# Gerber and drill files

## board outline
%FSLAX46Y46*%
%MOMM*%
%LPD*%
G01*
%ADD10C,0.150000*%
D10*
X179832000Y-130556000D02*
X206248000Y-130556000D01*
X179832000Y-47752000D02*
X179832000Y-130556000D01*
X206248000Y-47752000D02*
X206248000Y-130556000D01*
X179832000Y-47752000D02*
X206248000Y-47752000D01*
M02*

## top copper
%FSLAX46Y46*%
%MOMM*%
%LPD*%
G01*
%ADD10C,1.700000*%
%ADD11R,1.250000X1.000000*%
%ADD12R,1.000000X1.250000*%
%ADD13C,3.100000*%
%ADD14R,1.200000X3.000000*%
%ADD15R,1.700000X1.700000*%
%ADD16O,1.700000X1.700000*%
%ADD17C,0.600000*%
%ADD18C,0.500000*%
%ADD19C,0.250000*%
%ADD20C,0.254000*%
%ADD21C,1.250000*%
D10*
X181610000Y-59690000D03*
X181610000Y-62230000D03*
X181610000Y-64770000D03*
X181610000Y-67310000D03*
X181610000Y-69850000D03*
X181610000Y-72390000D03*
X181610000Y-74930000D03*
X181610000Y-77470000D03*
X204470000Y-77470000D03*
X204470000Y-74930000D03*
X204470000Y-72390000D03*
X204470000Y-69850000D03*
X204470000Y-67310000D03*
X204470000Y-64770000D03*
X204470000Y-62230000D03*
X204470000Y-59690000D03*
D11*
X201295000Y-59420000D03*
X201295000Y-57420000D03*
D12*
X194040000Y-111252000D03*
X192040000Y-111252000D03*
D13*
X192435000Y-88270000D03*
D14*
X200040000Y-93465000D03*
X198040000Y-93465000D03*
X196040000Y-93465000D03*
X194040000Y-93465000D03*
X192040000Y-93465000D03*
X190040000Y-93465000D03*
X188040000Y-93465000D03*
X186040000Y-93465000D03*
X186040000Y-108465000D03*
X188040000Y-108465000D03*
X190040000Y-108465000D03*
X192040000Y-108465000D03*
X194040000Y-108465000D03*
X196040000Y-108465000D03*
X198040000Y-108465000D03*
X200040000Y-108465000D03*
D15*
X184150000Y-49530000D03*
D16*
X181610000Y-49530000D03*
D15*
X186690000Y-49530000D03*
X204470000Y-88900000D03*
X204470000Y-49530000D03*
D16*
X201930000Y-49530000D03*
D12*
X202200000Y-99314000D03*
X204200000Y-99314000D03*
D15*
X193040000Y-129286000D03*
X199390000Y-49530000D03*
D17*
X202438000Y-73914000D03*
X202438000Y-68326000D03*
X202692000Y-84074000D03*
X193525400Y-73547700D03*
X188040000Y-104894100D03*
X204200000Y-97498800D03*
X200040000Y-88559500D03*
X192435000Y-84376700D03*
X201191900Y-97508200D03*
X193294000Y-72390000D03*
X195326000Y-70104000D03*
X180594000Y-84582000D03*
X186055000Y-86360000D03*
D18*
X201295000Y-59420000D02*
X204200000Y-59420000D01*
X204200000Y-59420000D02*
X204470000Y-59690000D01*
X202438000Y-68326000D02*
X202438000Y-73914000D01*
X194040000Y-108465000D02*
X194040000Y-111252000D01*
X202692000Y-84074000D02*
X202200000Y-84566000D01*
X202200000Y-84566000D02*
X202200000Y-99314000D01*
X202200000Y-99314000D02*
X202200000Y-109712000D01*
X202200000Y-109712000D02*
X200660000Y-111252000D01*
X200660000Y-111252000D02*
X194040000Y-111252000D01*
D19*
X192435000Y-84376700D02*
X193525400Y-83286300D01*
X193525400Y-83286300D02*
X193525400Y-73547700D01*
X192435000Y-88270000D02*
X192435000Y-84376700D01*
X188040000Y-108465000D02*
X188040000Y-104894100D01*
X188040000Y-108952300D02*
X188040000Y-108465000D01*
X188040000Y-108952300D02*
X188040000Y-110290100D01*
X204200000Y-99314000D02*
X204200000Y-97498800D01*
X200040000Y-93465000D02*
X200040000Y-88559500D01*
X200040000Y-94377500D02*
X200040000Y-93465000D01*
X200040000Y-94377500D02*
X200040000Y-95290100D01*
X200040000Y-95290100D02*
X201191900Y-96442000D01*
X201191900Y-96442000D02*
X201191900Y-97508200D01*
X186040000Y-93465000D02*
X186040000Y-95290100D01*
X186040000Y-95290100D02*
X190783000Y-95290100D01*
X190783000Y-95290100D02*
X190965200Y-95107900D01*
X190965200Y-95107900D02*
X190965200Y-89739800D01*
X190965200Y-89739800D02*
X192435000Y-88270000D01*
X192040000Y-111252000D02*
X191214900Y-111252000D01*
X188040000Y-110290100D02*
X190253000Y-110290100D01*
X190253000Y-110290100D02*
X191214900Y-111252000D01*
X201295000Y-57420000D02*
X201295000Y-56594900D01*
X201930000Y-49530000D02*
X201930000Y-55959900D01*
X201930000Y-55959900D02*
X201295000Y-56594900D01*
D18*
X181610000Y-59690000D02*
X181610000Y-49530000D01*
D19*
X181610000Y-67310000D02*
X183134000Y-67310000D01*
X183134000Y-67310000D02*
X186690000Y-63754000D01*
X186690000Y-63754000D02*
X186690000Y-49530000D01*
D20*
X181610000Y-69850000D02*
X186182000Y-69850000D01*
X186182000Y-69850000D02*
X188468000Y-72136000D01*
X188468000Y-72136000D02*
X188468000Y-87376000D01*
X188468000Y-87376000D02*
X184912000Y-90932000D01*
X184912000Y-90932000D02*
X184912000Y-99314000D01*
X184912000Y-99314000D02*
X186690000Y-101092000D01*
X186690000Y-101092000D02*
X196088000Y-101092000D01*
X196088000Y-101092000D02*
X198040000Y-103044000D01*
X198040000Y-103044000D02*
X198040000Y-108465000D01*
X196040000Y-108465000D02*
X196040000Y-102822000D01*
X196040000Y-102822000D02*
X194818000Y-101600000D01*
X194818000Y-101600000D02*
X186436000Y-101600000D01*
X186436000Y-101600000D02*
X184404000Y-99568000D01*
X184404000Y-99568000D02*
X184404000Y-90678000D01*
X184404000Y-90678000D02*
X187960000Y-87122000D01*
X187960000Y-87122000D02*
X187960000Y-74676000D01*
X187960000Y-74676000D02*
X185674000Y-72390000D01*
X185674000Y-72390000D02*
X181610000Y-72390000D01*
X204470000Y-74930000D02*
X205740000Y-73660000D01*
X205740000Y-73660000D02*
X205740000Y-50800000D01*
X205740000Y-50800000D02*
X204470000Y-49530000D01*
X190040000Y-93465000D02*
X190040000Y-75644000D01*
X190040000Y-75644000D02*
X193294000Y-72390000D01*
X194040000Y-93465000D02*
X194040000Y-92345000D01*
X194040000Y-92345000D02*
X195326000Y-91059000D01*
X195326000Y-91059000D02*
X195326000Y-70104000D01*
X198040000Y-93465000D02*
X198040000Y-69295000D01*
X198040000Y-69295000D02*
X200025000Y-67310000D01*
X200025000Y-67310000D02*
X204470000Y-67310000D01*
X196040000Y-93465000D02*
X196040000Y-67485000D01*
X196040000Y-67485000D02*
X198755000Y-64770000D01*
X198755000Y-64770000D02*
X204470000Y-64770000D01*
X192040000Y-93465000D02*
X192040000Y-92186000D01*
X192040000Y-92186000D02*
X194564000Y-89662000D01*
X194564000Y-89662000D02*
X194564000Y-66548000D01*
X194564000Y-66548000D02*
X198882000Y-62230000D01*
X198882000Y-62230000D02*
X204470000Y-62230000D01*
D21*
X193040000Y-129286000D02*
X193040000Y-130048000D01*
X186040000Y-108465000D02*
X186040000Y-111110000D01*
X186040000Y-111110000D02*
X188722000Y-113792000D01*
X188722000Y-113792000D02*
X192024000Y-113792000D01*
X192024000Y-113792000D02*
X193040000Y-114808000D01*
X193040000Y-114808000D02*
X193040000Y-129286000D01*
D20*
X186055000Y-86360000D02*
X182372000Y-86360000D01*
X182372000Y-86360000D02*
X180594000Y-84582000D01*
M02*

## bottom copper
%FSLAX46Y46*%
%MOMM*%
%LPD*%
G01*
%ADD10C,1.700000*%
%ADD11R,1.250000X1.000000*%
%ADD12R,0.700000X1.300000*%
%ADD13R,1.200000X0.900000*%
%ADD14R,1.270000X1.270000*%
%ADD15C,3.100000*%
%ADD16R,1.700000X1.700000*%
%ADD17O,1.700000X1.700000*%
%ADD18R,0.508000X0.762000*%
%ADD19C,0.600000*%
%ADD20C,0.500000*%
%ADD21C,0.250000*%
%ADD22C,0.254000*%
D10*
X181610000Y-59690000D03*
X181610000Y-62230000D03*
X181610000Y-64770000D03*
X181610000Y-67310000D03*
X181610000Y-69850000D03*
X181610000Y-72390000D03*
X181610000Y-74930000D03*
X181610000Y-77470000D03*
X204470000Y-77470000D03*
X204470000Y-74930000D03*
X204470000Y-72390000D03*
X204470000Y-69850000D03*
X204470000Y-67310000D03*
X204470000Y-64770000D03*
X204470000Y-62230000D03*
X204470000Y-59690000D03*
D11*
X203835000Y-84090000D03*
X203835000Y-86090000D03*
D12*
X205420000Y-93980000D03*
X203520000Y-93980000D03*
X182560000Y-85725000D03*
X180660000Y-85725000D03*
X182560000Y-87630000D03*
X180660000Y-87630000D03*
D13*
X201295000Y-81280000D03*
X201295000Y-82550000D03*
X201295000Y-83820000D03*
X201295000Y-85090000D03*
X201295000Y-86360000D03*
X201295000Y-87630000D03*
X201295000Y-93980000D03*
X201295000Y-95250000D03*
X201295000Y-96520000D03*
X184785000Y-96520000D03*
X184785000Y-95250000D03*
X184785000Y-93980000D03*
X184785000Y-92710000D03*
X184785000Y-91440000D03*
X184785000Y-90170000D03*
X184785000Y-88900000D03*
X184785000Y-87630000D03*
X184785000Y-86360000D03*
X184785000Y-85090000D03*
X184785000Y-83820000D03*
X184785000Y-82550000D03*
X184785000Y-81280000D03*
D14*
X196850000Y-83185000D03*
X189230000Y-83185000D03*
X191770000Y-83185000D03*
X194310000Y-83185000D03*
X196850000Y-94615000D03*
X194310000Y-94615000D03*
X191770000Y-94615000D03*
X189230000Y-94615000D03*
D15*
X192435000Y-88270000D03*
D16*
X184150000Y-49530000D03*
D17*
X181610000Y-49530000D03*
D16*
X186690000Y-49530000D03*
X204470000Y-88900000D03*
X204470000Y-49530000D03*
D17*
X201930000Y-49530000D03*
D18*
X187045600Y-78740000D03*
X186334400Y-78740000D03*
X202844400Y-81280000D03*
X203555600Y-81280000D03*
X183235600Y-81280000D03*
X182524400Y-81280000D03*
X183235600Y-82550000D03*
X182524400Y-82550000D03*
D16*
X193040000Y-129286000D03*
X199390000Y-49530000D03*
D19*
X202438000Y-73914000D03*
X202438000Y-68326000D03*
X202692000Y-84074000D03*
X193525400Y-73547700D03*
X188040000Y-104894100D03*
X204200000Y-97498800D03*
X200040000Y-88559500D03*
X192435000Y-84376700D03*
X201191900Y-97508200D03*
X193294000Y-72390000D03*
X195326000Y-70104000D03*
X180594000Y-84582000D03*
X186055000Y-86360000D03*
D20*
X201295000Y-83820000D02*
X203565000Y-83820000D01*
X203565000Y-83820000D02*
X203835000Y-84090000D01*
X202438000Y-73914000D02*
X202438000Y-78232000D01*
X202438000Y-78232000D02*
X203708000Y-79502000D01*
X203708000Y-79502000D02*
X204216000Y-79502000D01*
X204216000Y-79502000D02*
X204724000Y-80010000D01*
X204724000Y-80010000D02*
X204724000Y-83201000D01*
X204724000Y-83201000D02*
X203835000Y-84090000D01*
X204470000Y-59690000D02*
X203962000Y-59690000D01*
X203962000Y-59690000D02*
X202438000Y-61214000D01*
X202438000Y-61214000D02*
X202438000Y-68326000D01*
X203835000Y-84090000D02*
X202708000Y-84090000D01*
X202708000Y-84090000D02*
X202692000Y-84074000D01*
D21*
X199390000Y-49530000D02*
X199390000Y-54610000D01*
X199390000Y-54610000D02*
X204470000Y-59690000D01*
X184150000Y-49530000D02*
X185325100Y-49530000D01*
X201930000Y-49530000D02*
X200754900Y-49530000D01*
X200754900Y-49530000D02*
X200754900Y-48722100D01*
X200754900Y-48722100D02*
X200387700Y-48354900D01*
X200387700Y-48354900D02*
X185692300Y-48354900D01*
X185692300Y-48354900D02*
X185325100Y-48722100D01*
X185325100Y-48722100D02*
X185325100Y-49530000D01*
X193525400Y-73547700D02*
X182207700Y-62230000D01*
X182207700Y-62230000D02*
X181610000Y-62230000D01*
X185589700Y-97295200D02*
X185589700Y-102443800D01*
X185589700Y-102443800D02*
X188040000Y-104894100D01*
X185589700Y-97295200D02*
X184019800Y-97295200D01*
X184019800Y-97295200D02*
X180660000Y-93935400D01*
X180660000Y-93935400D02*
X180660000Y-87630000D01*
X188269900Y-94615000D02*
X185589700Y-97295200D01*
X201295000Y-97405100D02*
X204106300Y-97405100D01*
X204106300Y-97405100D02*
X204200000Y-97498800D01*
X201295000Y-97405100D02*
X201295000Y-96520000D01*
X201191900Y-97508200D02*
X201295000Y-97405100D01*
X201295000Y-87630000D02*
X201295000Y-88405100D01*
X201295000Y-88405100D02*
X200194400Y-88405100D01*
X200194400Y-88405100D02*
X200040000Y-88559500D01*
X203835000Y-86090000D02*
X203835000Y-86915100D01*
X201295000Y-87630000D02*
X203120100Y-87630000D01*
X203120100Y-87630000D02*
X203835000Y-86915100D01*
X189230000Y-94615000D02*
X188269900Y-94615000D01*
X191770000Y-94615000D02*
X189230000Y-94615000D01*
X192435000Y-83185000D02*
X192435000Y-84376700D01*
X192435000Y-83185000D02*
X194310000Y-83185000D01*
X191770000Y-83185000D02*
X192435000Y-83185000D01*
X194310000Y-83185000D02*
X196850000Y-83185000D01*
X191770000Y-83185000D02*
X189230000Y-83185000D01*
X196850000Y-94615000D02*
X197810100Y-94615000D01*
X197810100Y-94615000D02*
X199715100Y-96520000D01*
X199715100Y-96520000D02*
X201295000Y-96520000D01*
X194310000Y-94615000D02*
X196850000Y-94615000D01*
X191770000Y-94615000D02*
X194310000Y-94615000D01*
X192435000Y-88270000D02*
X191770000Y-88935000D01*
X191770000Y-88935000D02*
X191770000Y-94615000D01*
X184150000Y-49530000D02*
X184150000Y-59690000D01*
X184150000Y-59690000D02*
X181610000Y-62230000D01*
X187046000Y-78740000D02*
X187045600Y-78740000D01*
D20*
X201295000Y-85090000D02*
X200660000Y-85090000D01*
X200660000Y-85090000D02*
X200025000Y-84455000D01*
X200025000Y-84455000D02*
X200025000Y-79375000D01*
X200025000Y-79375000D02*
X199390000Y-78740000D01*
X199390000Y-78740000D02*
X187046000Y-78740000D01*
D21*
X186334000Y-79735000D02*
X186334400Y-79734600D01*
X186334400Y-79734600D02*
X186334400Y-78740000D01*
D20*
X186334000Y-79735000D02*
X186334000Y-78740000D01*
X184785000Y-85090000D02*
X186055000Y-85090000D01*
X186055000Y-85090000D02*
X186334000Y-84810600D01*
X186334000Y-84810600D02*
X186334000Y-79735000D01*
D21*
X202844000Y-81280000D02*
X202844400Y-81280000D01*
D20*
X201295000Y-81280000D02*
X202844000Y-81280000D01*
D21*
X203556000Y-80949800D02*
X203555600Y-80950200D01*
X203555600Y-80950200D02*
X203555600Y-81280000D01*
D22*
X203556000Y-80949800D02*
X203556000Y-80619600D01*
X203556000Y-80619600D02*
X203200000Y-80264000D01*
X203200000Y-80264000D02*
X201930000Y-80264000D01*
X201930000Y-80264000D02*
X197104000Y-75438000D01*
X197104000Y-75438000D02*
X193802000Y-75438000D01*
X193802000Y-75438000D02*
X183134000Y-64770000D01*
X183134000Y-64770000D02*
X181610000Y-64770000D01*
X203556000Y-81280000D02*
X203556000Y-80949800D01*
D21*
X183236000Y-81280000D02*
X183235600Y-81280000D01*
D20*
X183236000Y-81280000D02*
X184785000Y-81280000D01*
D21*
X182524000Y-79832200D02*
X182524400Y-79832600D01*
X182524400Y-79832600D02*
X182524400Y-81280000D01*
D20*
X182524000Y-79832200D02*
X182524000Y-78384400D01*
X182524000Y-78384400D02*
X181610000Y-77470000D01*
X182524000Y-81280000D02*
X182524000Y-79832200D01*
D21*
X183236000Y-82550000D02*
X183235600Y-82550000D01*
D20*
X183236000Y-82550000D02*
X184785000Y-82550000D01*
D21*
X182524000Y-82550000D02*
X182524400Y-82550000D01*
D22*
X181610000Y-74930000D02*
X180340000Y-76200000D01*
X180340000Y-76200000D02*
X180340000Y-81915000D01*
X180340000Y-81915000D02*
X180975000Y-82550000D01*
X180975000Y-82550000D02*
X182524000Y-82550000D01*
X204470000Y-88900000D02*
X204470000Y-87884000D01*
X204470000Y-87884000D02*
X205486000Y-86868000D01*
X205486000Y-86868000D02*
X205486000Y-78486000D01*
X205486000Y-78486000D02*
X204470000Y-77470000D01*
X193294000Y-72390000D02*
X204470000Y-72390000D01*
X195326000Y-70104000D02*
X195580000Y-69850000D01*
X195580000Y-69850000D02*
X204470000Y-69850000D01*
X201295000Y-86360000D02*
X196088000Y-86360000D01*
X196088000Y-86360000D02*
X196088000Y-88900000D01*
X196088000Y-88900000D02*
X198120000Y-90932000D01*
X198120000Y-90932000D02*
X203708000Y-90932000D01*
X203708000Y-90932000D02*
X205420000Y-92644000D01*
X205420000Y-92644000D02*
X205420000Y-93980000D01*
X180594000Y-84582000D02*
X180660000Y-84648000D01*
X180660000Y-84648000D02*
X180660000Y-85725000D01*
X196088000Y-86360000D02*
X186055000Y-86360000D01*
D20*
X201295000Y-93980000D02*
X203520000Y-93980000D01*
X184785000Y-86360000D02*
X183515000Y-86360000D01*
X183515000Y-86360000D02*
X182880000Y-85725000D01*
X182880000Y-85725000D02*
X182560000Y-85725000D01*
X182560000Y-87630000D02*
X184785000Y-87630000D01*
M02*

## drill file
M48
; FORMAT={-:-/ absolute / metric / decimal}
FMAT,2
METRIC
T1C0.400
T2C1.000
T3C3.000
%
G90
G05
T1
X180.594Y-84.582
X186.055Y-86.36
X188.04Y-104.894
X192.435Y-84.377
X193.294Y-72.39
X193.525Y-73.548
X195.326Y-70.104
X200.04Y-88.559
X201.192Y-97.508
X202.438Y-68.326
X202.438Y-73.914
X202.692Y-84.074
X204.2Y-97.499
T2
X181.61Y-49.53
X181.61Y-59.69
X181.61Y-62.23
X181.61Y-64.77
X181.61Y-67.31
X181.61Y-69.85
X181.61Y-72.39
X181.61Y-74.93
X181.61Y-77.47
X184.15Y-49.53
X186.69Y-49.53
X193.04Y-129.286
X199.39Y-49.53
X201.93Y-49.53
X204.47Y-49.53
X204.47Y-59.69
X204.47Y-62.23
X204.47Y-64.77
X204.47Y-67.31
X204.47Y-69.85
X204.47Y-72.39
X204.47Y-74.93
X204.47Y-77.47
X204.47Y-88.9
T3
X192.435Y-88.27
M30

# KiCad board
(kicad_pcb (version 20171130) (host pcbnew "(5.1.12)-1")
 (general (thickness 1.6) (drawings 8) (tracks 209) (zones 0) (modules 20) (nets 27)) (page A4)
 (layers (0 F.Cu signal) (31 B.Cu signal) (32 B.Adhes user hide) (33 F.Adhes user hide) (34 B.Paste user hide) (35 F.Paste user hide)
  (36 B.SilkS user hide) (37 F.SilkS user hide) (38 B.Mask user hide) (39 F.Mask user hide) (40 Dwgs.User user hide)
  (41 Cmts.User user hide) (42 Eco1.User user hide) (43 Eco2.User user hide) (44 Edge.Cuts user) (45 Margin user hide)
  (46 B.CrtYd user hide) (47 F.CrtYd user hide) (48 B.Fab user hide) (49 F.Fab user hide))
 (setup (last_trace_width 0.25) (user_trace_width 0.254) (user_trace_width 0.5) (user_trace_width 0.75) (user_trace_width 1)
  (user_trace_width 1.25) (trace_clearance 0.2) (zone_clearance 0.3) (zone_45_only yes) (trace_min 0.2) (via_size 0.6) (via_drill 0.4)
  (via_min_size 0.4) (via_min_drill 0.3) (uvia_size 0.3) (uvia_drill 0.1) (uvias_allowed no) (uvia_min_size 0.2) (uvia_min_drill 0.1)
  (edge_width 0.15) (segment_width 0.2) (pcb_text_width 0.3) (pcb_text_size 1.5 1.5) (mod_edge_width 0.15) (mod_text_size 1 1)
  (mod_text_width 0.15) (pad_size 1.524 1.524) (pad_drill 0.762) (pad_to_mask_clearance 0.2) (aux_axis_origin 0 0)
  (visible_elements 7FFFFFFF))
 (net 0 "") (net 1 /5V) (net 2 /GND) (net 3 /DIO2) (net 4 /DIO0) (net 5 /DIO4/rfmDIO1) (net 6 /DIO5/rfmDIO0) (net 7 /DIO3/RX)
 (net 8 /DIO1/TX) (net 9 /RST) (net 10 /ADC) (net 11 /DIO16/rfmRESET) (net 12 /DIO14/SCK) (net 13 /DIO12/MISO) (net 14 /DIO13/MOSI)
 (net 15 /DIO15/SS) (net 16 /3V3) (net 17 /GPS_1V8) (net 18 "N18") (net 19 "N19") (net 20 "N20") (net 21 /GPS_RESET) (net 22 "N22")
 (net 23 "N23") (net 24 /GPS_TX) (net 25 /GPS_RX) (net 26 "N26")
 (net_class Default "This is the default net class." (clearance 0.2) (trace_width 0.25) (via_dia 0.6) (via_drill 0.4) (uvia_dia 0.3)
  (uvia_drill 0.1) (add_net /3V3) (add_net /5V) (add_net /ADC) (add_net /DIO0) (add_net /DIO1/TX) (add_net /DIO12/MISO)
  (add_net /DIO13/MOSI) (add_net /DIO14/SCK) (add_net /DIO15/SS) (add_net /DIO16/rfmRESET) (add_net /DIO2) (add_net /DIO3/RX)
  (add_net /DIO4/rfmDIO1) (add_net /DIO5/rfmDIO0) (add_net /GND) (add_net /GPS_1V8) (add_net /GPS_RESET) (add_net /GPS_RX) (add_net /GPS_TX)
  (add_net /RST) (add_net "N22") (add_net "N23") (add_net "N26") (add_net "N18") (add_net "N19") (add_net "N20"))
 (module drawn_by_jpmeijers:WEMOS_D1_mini (layer F.Cu) (at 193.04 68.58)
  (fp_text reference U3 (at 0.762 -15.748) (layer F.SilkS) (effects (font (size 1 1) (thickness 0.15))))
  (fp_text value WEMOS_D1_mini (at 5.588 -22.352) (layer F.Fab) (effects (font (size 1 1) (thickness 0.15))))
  (pad 1 thru_hole circle (at -11.43 -8.89) (size 1.7 1.7) (drill 1) (layers *.Cu *.Mask) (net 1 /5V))
  (pad 2 thru_hole circle (at -11.43 -6.35) (size 1.7 1.7) (drill 1) (layers *.Cu *.Mask) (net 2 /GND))
  (pad 3 thru_hole circle (at -11.43 -3.81) (size 1.7 1.7) (drill 1) (layers *.Cu *.Mask) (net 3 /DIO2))
  (pad 4 thru_hole circle (at -11.43 -1.27) (size 1.7 1.7) (drill 1) (layers *.Cu *.Mask) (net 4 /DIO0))
  (pad 5 thru_hole circle (at -11.43 1.27) (size 1.7 1.7) (drill 1) (layers *.Cu *.Mask) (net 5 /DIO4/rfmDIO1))
  (pad 6 thru_hole circle (at -11.43 3.81) (size 1.7 1.7) (drill 1) (layers *.Cu *.Mask) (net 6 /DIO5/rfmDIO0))
  (pad 7 thru_hole circle (at -11.43 6.35) (size 1.7 1.7) (drill 1) (layers *.Cu *.Mask) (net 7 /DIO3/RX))
  (pad 8 thru_hole circle (at -11.43 8.89) (size 1.7 1.7) (drill 1) (layers *.Cu *.Mask) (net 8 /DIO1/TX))
  (pad 9 thru_hole circle (at 11.43 8.89) (size 1.7 1.7) (drill 1) (layers *.Cu *.Mask) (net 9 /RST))
  (pad 10 thru_hole circle (at 11.43 6.35) (size 1.7 1.7) (drill 1) (layers *.Cu *.Mask) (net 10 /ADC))
  (pad 11 thru_hole circle (at 11.43 3.81) (size 1.7 1.7) (drill 1) (layers *.Cu *.Mask) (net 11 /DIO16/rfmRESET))
  (pad 12 thru_hole circle (at 11.43 1.27) (size 1.7 1.7) (drill 1) (layers *.Cu *.Mask) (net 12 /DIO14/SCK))
  (pad 13 thru_hole circle (at 11.43 -1.27) (size 1.7 1.7) (drill 1) (layers *.Cu *.Mask) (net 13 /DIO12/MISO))
  (pad 14 thru_hole circle (at 11.43 -3.81) (size 1.7 1.7) (drill 1) (layers *.Cu *.Mask) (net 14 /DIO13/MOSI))
  (pad 15 thru_hole circle (at 11.43 -6.35) (size 1.7 1.7) (drill 1) (layers *.Cu *.Mask) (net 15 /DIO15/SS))
  (pad 16 thru_hole circle (at 11.43 -8.89) (size 1.7 1.7) (drill 1) (layers *.Cu *.Mask) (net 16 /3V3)))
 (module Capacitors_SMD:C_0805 (layer F.Cu) (at 201.295 58.42 90)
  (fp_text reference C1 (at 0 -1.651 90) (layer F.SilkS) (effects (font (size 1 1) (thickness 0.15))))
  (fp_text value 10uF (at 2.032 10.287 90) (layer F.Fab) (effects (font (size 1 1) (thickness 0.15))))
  (pad 1 smd rect (at -1 0 90) (size 1 1.25) (layers F.Cu F.Paste F.Mask) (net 16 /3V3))
  (pad 2 smd rect (at 1 0 90) (size 1 1.25) (layers F.Cu F.Paste F.Mask) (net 2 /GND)))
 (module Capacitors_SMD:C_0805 (layer B.Cu) (at 203.835 85.09 270)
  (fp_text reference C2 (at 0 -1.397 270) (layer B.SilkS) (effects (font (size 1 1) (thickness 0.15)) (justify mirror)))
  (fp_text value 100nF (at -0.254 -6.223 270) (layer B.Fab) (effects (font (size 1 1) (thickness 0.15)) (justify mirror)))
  (pad 1 smd rect (at -1 0 270) (size 1 1.25) (layers B.Cu B.Paste B.Mask) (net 16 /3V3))
  (pad 2 smd rect (at 1 0 270) (size 1 1.25) (layers B.Cu B.Paste B.Mask) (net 2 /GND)))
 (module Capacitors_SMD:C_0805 (layer F.Cu) (at 193.04 111.252 180)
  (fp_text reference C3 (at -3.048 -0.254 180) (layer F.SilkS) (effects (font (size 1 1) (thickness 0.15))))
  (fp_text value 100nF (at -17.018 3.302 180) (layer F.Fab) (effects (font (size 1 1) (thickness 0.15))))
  (pad 1 smd rect (at -1 0 180) (size 1 1.25) (layers F.Cu F.Paste F.Mask) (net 16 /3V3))
  (pad 2 smd rect (at 1 0 180) (size 1 1.25) (layers F.Cu F.Paste F.Mask) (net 2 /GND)))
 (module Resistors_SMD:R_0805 (layer B.Cu) (at 204.47 93.98 180)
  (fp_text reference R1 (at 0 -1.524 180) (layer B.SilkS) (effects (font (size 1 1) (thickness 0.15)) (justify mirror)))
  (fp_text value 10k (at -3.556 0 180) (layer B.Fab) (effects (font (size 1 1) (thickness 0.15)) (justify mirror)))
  (pad 1 smd rect (at -0.95 0 180) (size 0.7 1.3) (layers B.Cu B.Paste B.Mask) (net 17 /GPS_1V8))
  (pad 2 smd rect (at 0.95 0 180) (size 0.7 1.3) (layers B.Cu B.Paste B.Mask) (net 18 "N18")))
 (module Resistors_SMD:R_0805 (layer B.Cu) (at 181.61 85.725 180)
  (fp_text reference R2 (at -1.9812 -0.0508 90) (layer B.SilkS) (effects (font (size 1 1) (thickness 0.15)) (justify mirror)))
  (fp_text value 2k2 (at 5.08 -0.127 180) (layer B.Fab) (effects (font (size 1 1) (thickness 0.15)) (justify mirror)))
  (pad 1 smd rect (at -0.95 0 180) (size 0.7 1.3) (layers B.Cu B.Paste B.Mask) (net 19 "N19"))
  (pad 2 smd rect (at 0.95 0 180) (size 0.7 1.3) (layers B.Cu B.Paste B.Mask) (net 17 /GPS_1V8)))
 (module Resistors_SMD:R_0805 (layer B.Cu) (at 181.61 87.63 180)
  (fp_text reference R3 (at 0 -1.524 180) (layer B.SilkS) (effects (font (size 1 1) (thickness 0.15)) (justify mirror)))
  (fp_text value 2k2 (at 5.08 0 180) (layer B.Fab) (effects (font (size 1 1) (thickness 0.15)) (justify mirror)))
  (pad 1 smd rect (at -0.95 0 180) (size 0.7 1.3) (layers B.Cu B.Paste B.Mask) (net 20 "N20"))
  (pad 2 smd rect (at 0.95 0 180) (size 0.7 1.3) (layers B.Cu B.Paste B.Mask) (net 2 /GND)))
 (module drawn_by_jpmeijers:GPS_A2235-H (layer B.Cu) (at 201.295 97.79 180)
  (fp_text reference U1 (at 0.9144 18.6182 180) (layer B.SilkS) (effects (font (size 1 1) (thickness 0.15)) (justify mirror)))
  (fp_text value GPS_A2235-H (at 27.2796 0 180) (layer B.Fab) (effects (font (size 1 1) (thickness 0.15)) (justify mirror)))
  (pad 1 smd rect (at 0 16.51 180) (size 1.2 0.9) (layers B.Cu B.Paste B.Mask) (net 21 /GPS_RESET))
  (pad 2 smd rect (at 0 15.24 180) (size 1.2 0.9) (layers B.Cu B.Paste B.Mask))
  (pad 3 smd rect (at 0 13.97 180) (size 1.2 0.9) (layers B.Cu B.Paste B.Mask) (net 16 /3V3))
  (pad 4 smd rect (at 0 12.7 180) (size 1.2 0.9) (layers B.Cu B.Paste B.Mask) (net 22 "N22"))
  (pad 5 smd rect (at 0 11.43 180) (size 1.2 0.9) (layers B.Cu B.Paste B.Mask) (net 17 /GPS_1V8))
  (pad 6 smd rect (at 0 10.16 180) (size 1.2 0.9) (layers B.Cu B.Paste B.Mask) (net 2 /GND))
  (pad 7 smd rect (at 0 3.81 180) (size 1.2 0.9) (layers B.Cu B.Paste B.Mask) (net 18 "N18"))
  (pad 8 smd rect (at 0 2.54 180) (size 1.2 0.9) (layers B.Cu B.Paste B.Mask))
  (pad 9 smd rect (at 0 1.27 180) (size 1.2 0.9) (layers B.Cu B.Paste B.Mask) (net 2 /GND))
  (pad 10 smd rect (at 16.51 1.27 180) (size 1.2 0.9) (layers B.Cu B.Paste B.Mask))
  (pad 11 smd rect (at 16.51 2.54 180) (size 1.2 0.9) (layers B.Cu B.Paste B.Mask))
  (pad 12 smd rect (at 16.51 3.81 180) (size 1.2 0.9) (layers B.Cu B.Paste B.Mask))
  (pad 13 smd rect (at 16.51 5.08 180) (size 1.2 0.9) (layers B.Cu B.Paste B.Mask))
  (pad 14 smd rect (at 16.51 6.35 180) (size 1.2 0.9) (layers B.Cu B.Paste B.Mask))
  (pad 15 smd rect (at 16.51 7.62 180) (size 1.2 0.9) (layers B.Cu B.Paste B.Mask))
  (pad 16 smd rect (at 16.51 8.89 180) (size 1.2 0.9) (layers B.Cu B.Paste B.Mask))
  (pad 17 smd rect (at 16.51 10.16 180) (size 1.2 0.9) (layers B.Cu B.Paste B.Mask) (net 20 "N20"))
  (pad 18 smd rect (at 16.51 11.43 180) (size 1.2 0.9) (layers B.Cu B.Paste B.Mask) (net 19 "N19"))
  (pad 19 smd rect (at 16.51 12.7 180) (size 1.2 0.9) (layers B.Cu B.Paste B.Mask) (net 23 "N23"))
  (pad 20 smd rect (at 16.51 13.97 180) (size 1.2 0.9) (layers B.Cu B.Paste B.Mask))
  (pad 21 smd rect (at 16.51 15.24 180) (size 1.2 0.9) (layers B.Cu B.Paste B.Mask) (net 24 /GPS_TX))
  (pad 22 smd rect (at 16.51 16.51 180) (size 1.2 0.9) (layers B.Cu B.Paste B.Mask) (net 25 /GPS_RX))
  (pad 23 smd rect (at 4.445 14.605 180) (size 1.27 1.27) (layers B.Cu B.Paste B.Mask) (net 2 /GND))
  (pad 26 smd rect (at 12.065 14.605 180) (size 1.27 1.27) (layers B.Cu B.Paste B.Mask) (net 2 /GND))
  (pad 25 smd rect (at 9.525 14.605 180) (size 1.27 1.27) (layers B.Cu B.Paste B.Mask) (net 2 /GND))
  (pad 24 smd rect (at 6.985 14.605 180) (size 1.27 1.27) (layers B.Cu B.Paste B.Mask) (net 2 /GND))
  (pad 27 smd rect (at 4.445 3.175 180) (size 1.27 1.27) (layers B.Cu B.Paste B.Mask) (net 2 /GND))
  (pad 28 smd rect (at 6.985 3.175 180) (size 1.27 1.27) (layers B.Cu B.Paste B.Mask) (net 2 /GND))
  (pad 29 smd rect (at 9.525 3.175 180) (size 1.27 1.27) (layers B.Cu B.Paste B.Mask) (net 2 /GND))
  (pad 30 smd rect (at 12.065 3.175 180) (size 1.27 1.27) (layers B.Cu B.Paste B.Mask) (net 2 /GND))
  (pad 31 thru_hole circle (at 8.86 9.52 180) (size 3.1 3.1) (drill 3) (layers *.Cu *.Mask B.SilkS) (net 2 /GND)))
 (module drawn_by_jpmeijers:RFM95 (layer F.Cu) (at 193.04 100.965 270)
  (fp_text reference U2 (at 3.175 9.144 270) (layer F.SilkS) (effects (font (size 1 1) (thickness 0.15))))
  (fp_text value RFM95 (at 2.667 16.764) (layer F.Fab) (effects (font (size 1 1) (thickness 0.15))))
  (pad 1 smd rect (at -7.5 -7 270) (size 3 1.2) (layers F.Cu F.Paste F.Mask) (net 2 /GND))
  (pad 2 smd rect (at -7.5 -5 270) (size 3 1.2) (layers F.Cu F.Paste F.Mask) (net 13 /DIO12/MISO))
  (pad 3 smd rect (at -7.5 -3 270) (size 3 1.2) (layers F.Cu F.Paste F.Mask) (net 14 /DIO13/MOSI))
  (pad 4 smd rect (at -7.5 -1 270) (size 3 1.2) (layers F.Cu F.Paste F.Mask) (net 12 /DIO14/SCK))
  (pad 5 smd rect (at -7.5 1 270) (size 3 1.2) (layers F.Cu F.Paste F.Mask) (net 15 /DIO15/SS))
  (pad 6 smd rect (at -7.5 3 270) (size 3 1.2) (layers F.Cu F.Paste F.Mask) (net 11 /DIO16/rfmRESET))
  (pad 7 smd rect (at -7.5 5 270) (size 3 1.2) (layers F.Cu F.Paste F.Mask))
  (pad 8 smd rect (at -7.5 7 270) (size 3 1.2) (layers F.Cu F.Paste F.Mask) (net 2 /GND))
  (pad 9 smd rect (at 7.5 7 270) (size 3 1.2) (layers F.Cu F.Paste F.Mask) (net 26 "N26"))
  (pad 10 smd rect (at 7.5 5 270) (size 3 1.2) (layers F.Cu F.Paste F.Mask) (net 2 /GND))
  (pad 11 smd rect (at 7.5 3 270) (size 3 1.2) (layers F.Cu F.Paste F.Mask))
  (pad 12 smd rect (at 7.5 1 270) (size 3 1.2) (layers F.Cu F.Paste F.Mask))
  (pad 13 smd rect (at 7.5 -1 270) (size 3 1.2) (layers F.Cu F.Paste F.Mask) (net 16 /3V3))
  (pad 14 smd rect (at 7.5 -3 270) (size 3 1.2) (layers F.Cu F.Paste F.Mask) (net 6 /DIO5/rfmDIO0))
  (pad 15 smd rect (at 7.5 -5 270) (size 3 1.2) (layers F.Cu F.Paste F.Mask) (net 5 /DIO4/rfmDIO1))
  (pad 16 smd rect (at 7.5 -7 270) (size 3 1.2) (layers F.Cu F.Paste F.Mask)))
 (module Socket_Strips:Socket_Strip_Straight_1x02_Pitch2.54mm (layer F.Cu) (at 184.15 49.53 270)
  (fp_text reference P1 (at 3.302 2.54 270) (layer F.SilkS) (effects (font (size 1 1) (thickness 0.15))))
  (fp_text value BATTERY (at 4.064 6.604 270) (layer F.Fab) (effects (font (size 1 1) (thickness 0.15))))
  (pad 1 thru_hole rect (at 0 0 270) (size 1.7 1.7) (drill 1) (layers *.Cu *.Mask) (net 2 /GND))
  (pad 2 thru_hole oval (at 0 2.54 270) (size 1.7 1.7) (drill 1) (layers *.Cu *.Mask) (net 1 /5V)))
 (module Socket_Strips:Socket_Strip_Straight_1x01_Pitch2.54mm (layer F.Cu) (at 186.69 49.53)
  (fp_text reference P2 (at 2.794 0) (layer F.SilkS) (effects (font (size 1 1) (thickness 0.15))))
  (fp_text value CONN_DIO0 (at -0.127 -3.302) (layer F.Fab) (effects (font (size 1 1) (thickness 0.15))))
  (pad 1 thru_hole rect (at 0 0) (size 1.7 1.7) (drill 1) (layers *.Cu *.Mask) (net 4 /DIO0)))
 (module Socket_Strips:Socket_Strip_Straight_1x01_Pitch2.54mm (layer F.Cu) (at 204.47 88.9)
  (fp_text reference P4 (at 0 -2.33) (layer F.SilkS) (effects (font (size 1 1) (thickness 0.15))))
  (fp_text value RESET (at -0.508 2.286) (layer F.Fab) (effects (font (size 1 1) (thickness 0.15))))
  (pad 1 thru_hole rect (at 0 0) (size 1.7 1.7) (drill 1) (layers *.Cu *.Mask) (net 9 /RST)))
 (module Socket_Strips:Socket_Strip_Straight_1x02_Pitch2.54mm (layer F.Cu) (at 204.47 49.53 270)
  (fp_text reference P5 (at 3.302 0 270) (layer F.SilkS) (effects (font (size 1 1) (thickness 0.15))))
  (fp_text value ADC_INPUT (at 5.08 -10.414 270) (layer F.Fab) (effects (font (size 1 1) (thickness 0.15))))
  (pad 1 thru_hole rect (at 0 0 270) (size 1.7 1.7) (drill 1) (layers *.Cu *.Mask) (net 10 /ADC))
  (pad 2 thru_hole oval (at 0 2.54 270) (size 1.7 1.7) (drill 1) (layers *.Cu *.Mask) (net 2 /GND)))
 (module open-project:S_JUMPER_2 (layer B.Cu) (at 186.69 78.74 180)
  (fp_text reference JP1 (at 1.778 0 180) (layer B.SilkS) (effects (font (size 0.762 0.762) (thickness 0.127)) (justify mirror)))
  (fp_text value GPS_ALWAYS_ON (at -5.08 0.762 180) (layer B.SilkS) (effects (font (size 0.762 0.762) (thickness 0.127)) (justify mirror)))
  (pad 1 smd rect (at -0.3556 0 180) (size 0.508 0.762) (layers B.Cu B.Paste B.Mask) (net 22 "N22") (clearance 0.2032))
  (pad 2 smd rect (at 0.3556 0 180) (size 0.508 0.762) (layers B.Cu B.Paste B.Mask) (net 23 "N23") (clearance 0.2032)))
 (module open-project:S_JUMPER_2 (layer B.Cu) (at 203.2 81.28)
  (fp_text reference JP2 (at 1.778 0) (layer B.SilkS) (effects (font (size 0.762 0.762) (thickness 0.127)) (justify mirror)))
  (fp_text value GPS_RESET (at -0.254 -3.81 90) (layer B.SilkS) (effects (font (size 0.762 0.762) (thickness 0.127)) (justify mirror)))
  (pad 1 smd rect (at -0.3556 0) (size 0.508 0.762) (layers B.Cu B.Paste B.Mask) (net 21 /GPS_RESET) (clearance 0.2032))
  (pad 2 smd rect (at 0.3556 0) (size 0.508 0.762) (layers B.Cu B.Paste B.Mask) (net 3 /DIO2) (clearance 0.2032)))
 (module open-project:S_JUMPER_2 (layer B.Cu) (at 182.88 81.28 180)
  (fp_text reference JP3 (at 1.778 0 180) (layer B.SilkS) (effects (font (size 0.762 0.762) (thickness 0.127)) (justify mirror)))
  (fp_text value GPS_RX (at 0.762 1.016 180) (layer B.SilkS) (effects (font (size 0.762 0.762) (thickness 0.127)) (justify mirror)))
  (pad 1 smd rect (at -0.3556 0 180) (size 0.508 0.762) (layers B.Cu B.Paste B.Mask) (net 25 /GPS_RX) (clearance 0.2032))
  (pad 2 smd rect (at 0.3556 0 180) (size 0.508 0.762) (layers B.Cu B.Paste B.Mask) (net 8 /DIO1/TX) (clearance 0.2032)))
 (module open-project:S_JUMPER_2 (layer B.Cu) (at 182.88 82.55 180)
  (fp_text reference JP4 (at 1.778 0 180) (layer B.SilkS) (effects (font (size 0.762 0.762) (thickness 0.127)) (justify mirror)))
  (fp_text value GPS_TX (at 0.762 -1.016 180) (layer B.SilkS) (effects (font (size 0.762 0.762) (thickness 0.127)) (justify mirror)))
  (pad 1 smd rect (at -0.3556 0 180) (size 0.508 0.762) (layers B.Cu B.Paste B.Mask) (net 24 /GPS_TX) (clearance 0.2032))
  (pad 2 smd rect (at 0.3556 0 180) (size 0.508 0.762) (layers B.Cu B.Paste B.Mask) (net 7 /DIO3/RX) (clearance 0.2032)))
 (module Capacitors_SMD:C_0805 (layer F.Cu) (at 203.2 99.314)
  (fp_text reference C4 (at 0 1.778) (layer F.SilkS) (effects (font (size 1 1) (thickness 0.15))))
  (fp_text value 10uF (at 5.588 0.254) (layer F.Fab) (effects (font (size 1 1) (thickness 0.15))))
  (pad 1 smd rect (at -1 0) (size 1 1.25) (layers F.Cu F.Paste F.Mask) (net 16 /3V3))
  (pad 2 smd rect (at 1 0) (size 1 1.25) (layers F.Cu F.Paste F.Mask) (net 2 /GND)))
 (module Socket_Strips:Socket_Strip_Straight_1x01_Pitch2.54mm (layer F.Cu) (at 193.04 129.286)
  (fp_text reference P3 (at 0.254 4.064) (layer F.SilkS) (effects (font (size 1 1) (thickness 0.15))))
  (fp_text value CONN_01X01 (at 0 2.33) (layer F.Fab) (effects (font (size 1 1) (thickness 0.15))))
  (pad 1 thru_hole rect (at 0 0) (size 1.7 1.7) (drill 1) (layers *.Cu *.Mask) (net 26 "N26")))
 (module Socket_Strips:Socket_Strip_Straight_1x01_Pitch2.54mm (layer F.Cu) (at 199.39 49.53)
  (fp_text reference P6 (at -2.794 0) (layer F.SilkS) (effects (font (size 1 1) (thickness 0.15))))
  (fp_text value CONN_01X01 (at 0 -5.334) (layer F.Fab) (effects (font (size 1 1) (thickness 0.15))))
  (pad 1 thru_hole rect (at 0 0) (size 1.7 1.7) (drill 1) (layers *.Cu *.Mask) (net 16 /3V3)))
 (gr_line (start 179.832 130.556) (end 206.248 130.556) (angle 90) (layer Edge.Cuts) (width 0.15))
 (gr_line (start 179.832 47.752) (end 179.832 130.556) (angle 90) (layer Edge.Cuts) (width 0.15))
 (gr_line (start 206.248 47.752) (end 206.248 130.556) (angle 90) (layer Edge.Cuts) (width 0.15))
 (gr_line (start 179.832 47.752) (end 206.248 47.752) (angle 90) (layer Edge.Cuts) (width 0.15))
 (segment (start 201.295 83.82) (end 203.565 83.82) (width 0.5) (layer B.Cu) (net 16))
 (segment (start 203.565 83.82) (end 203.835 84.09) (width 0.5) (layer B.Cu) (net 16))
 (segment (start 201.295 59.42) (end 204.2 59.42) (width 0.5) (layer F.Cu) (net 16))
 (segment (start 204.2 59.42) (end 204.47 59.69) (width 0.5) (layer F.Cu) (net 16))
 (segment (start 202.438 73.914) (end 202.438 78.232) (width 0.5) (layer B.Cu) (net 16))
 (segment (start 202.438 78.232) (end 203.708 79.502) (width 0.5) (layer B.Cu) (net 16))
 (segment (start 203.708 79.502) (end 204.216 79.502) (width 0.5) (layer B.Cu) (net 16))
 (segment (start 204.216 79.502) (end 204.724 80.01) (width 0.5) (layer B.Cu) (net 16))
 (segment (start 204.724 80.01) (end 204.724 83.201) (width 0.5) (layer B.Cu) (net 16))
 (segment (start 204.724 83.201) (end 203.835 84.09) (width 0.5) (layer B.Cu) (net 16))
 (segment (start 202.438 68.326) (end 202.438 73.914) (width 0.5) (layer F.Cu) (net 16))
 (segment (start 204.47 59.69) (end 203.962 59.69) (width 0.5) (layer B.Cu) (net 16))
 (segment (start 203.962 59.69) (end 202.438 61.214) (width 0.5) (layer B.Cu) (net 16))
 (segment (start 202.438 61.214) (end 202.438 68.326) (width 0.5) (layer B.Cu) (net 16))
 (segment (start 194.04 108.465) (end 194.04 111.252) (width 0.5) (layer F.Cu) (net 16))
 (segment (start 203.835 84.09) (end 202.708 84.09) (width 0.5) (layer B.Cu) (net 16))
 (segment (start 202.708 84.09) (end 202.692 84.074) (width 0.5) (layer B.Cu) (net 16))
 (segment (start 202.692 84.074) (end 202.2 84.566) (width 0.5) (layer F.Cu) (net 16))
 (segment (start 202.2 84.566) (end 202.2 99.314) (width 0.5) (layer F.Cu) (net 16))
 (segment (start 202.2 99.314) (end 202.2 109.712) (width 0.5) (layer F.Cu) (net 16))
 (segment (start 202.2 109.712) (end 200.66 111.252) (width 0.5) (layer F.Cu) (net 16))
 (segment (start 200.66 111.252) (end 194.04 111.252) (width 0.5) (layer F.Cu) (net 16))
 (segment (start 199.39 49.53) (end 199.39 54.61) (width 0.25) (layer B.Cu) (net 16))
 (segment (start 199.39 54.61) (end 204.47 59.69) (width 0.25) (layer B.Cu) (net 16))
 (via (at 202.438 73.914) (size 0.6) (layers F.Cu B.Cu) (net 16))
 (via (at 202.438 68.326) (size 0.6) (layers F.Cu B.Cu) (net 16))
 (via (at 202.692 84.074) (size 0.6) (layers F.Cu B.Cu) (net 16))
 (segment (start 184.15 49.53) (end 185.3251 49.53) (width 0.25) (layer B.Cu) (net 2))
 (segment (start 201.93 49.53) (end 200.7549 49.53) (width 0.25) (layer B.Cu) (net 2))
 (segment (start 200.7549 49.53) (end 200.7549 48.7221) (width 0.25) (layer B.Cu) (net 2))
 (segment (start 200.7549 48.7221) (end 200.3877 48.3549) (width 0.25) (layer B.Cu) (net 2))
 (segment (start 200.3877 48.3549) (end 185.6923 48.3549) (width 0.25) (layer B.Cu) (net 2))
 (segment (start 185.6923 48.3549) (end 185.3251 48.7221) (width 0.25) (layer B.Cu) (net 2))
 (segment (start 185.3251 48.7221) (end 185.3251 49.53) (width 0.25) (layer B.Cu) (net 2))
 (segment (start 192.435 84.3767) (end 193.5254 83.2863) (width 0.25) (layer F.Cu) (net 2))
 (segment (start 193.5254 83.2863) (end 193.5254 73.5477) (width 0.25) (layer F.Cu) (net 2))
 (segment (start 192.435 88.27) (end 192.435 84.3767) (width 0.25) (layer F.Cu) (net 2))
 (segment (start 193.5254 73.5477) (end 182.2077 62.23) (width 0.25) (layer B.Cu) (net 2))
 (segment (start 182.2077 62.23) (end 181.61 62.23) (width 0.25) (layer B.Cu) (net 2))
 (segment (start 188.04 108.465) (end 188.04 104.8941) (width 0.25) (layer F.Cu) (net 2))
 (segment (start 185.5897 97.2952) (end 185.5897 102.4438) (width 0.25) (layer B.Cu) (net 2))
 (segment (start 185.5897 102.4438) (end 188.04 104.8941) (width 0.25) (layer B.Cu) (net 2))
 (segment (start 185.5897 97.2952) (end 184.0198 97.2952) (width 0.25) (layer B.Cu) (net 2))
 (segment (start 184.0198 97.2952) (end 180.66 93.9354) (width 0.25) (layer B.Cu) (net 2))
 (segment (start 180.66 93.9354) (end 180.66 87.63) (width 0.25) (layer B.Cu) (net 2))
 (segment (start 188.2699 94.615) (end 185.5897 97.2952) (width 0.25) (layer B.Cu) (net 2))
 (segment (start 188.04 108.9523) (end 188.04 108.465) (width 0.25) (layer F.Cu) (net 2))
 (segment (start 188.04 108.9523) (end 188.04 110.2901) (width 0.25) (layer F.Cu) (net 2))
 (segment (start 204.2 99.314) (end 204.2 97.4988) (width 0.25) (layer F.Cu) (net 2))
 (segment (start 201.295 97.4051) (end 204.1063 97.4051) (width 0.25) (layer B.Cu) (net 2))
 (segment (start 204.1063 97.4051) (end 204.2 97.4988) (width 0.25) (layer B.Cu) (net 2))
 (segment (start 201.295 97.4051) (end 201.295 96.52) (width 0.25) (layer B.Cu) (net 2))
 (segment (start 201.1919 97.5082) (end 201.295 97.4051) (width 0.25) (layer B.Cu) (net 2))
 (segment (start 201.295 87.63) (end 201.295 88.4051) (width 0.25) (layer B.Cu) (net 2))
 (segment (start 200.04 93.465) (end 200.04 88.5595) (width 0.25) (layer F.Cu) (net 2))
 (segment (start 201.295 88.4051) (end 200.1944 88.4051) (width 0.25) (layer B.Cu) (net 2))
 (segment (start 200.1944 88.4051) (end 200.04 88.5595) (width 0.25) (layer B.Cu) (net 2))
 (segment (start 200.04 94.3775) (end 200.04 93.465) (width 0.25) (layer F.Cu) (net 2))
 (segment (start 200.04 94.3775) (end 200.04 95.2901) (width 0.25) (layer F.Cu) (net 2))
 (segment (start 203.835 86.09) (end 203.835 86.9151) (width 0.25) (layer B.Cu) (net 2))
 (segment (start 201.295 87.63) (end 203.1201 87.63) (width 0.25) (layer B.Cu) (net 2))
 (segment (start 203.1201 87.63) (end 203.835 86.9151) (width 0.25) (layer B.Cu) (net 2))
 (segment (start 189.23 94.615) (end 188.2699 94.615) (width 0.25) (layer B.Cu) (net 2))
 (segment (start 191.77 94.615) (end 189.23 94.615) (width 0.25) (layer B.Cu) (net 2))
 (segment (start 192.435 83.185) (end 192.435 84.3767) (width 0.25) (layer B.Cu) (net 2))
 (segment (start 192.435 83.185) (end 194.31 83.185) (width 0.25) (layer B.Cu) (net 2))
 (segment (start 191.77 83.185) (end 192.435 83.185) (width 0.25) (layer B.Cu) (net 2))
 (segment (start 194.31 83.185) (end 196.85 83.185) (width 0.25) (layer B.Cu) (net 2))
 (segment (start 191.77 83.185) (end 189.23 83.185) (width 0.25) (layer B.Cu) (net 2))
 (segment (start 196.85 94.615) (end 197.8101 94.615) (width 0.25) (layer B.Cu) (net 2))
 (segment (start 197.8101 94.615) (end 199.7151 96.52) (width 0.25) (layer B.Cu) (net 2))
 (segment (start 199.7151 96.52) (end 201.295 96.52) (width 0.25) (layer B.Cu) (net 2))
 (segment (start 194.31 94.615) (end 196.85 94.615) (width 0.25) (layer B.Cu) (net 2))
 (segment (start 191.77 94.615) (end 194.31 94.615) (width 0.25) (layer B.Cu) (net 2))
 (segment (start 192.435 88.27) (end 191.77 88.935) (width 0.25) (layer B.Cu) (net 2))
 (segment (start 191.77 88.935) (end 191.77 94.615) (width 0.25) (layer B.Cu) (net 2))
 (segment (start 200.04 95.2901) (end 201.1919 96.442) (width 0.25) (layer F.Cu) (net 2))
 (segment (start 201.1919 96.442) (end 201.1919 97.5082) (width 0.25) (layer F.Cu) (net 2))
 (segment (start 186.04 93.465) (end 186.04 95.2901) (width 0.25) (layer F.Cu) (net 2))
 (segment (start 186.04 95.2901) (end 190.783 95.2901) (width 0.25) (layer F.Cu) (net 2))
 (segment (start 190.783 95.2901) (end 190.9652 95.1079) (width 0.25) (layer F.Cu) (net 2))
 (segment (start 190.9652 95.1079) (end 190.9652 89.7398) (width 0.25) (layer F.Cu) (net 2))
 (segment (start 190.9652 89.7398) (end 192.435 88.27) (width 0.25) (layer F.Cu) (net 2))
 (segment (start 192.04 111.252) (end 191.2149 111.252) (width 0.25) (layer F.Cu) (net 2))
 (segment (start 188.04 110.2901) (end 190.253 110.2901) (width 0.25) (layer F.Cu) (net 2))
 (segment (start 190.253 110.2901) (end 191.2149 111.252) (width 0.25) (layer F.Cu) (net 2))
 (segment (start 184.15 49.53) (end 184.15 59.69) (width 0.25) (layer B.Cu) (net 2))
 (segment (start 184.15 59.69) (end 181.61 62.23) (width 0.25) (layer B.Cu) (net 2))
 (segment (start 201.295 57.42) (end 201.295 56.5949) (width 0.25) (layer F.Cu) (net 2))
 (segment (start 201.93 49.53) (end 201.93 55.9599) (width 0.25) (layer F.Cu) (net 2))
 (segment (start 201.93 55.9599) (end 201.295 56.5949) (width 0.25) (layer F.Cu) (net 2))
 (via (at 193.5254 73.5477) (size 0.6) (layers F.Cu B.Cu) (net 2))
 (via (at 188.04 104.8941) (size 0.6) (layers F.Cu B.Cu) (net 2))
 (via (at 204.2 97.4988) (size 0.6) (layers F.Cu B.Cu) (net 2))
 (via (at 200.04 88.5595) (size 0.6) (layers F.Cu B.Cu) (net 2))
 (via (at 192.435 84.3767) (size 0.6) (layers F.Cu B.Cu) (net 2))
 (via (at 201.1919 97.5082) (size 0.6) (layers F.Cu B.Cu) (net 2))
 (segment (start 187.046 78.74) (end 187.0456 78.74) (width 0.25) (layer B.Cu) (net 22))
 (segment (start 201.295 85.09) (end 200.66 85.09) (width 0.5) (layer B.Cu) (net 22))
 (segment (start 200.66 85.09) (end 200.025 84.455) (width 0.5) (layer B.Cu) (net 22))
 (segment (start 200.025 84.455) (end 200.025 79.375) (width 0.5) (layer B.Cu) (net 22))
 (segment (start 200.025 79.375) (end 199.39 78.74) (width 0.5) (layer B.Cu) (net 22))
 (segment (start 199.39 78.74) (end 187.046 78.74) (width 0.5) (layer B.Cu) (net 22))
 (segment (start 186.334 79.735) (end 186.3344 79.7346) (width 0.25) (layer B.Cu) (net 23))
 (segment (start 186.3344 79.7346) (end 186.3344 78.74) (width 0.25) (layer B.Cu) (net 23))
 (segment (start 186.334 79.735) (end 186.334 78.74) (width 0.5) (layer B.Cu) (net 23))
 (segment (start 184.785 85.09) (end 186.055 85.09) (width 0.5) (layer B.Cu) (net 23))
 (segment (start 186.055 85.09) (end 186.334 84.8106) (width 0.5) (layer B.Cu) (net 23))
 (segment (start 186.334 84.8106) (end 186.334 79.735) (width 0.5) (layer B.Cu) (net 23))
 (segment (start 202.844 81.28) (end 202.8444 81.28) (width 0.25) (layer B.Cu) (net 21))
 (segment (start 201.295 81.28) (end 202.844 81.28) (width 0.5) (layer B.Cu) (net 21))
 (segment (start 203.556 80.9498) (end 203.5556 80.9502) (width 0.25) (layer B.Cu) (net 3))
 (segment (start 203.5556 80.9502) (end 203.5556 81.28) (width 0.25) (layer B.Cu) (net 3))
 (segment (start 203.556 80.9498) (end 203.556 80.6196) (width 0.254) (layer B.Cu) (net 3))
 (segment (start 203.556 80.6196) (end 203.2 80.264) (width 0.254) (layer B.Cu) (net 3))
 (segment (start 203.2 80.264) (end 201.93 80.264) (width 0.254) (layer B.Cu) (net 3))
 (segment (start 201.93 80.264) (end 197.104 75.438) (width 0.254) (layer B.Cu) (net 3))
 (segment (start 197.104 75.438) (end 193.802 75.438) (width 0.254) (layer B.Cu) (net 3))
 (segment (start 193.802 75.438) (end 183.134 64.77) (width 0.254) (layer B.Cu) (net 3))
 (segment (start 183.134 64.77) (end 181.61 64.77) (width 0.254) (layer B.Cu) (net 3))
 (segment (start 203.556 81.28) (end 203.556 80.9498) (width 0.254) (layer B.Cu) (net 3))
 (segment (start 183.236 81.28) (end 183.2356 81.28) (width 0.25) (layer B.Cu) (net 25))
 (segment (start 183.236 81.28) (end 184.785 81.28) (width 0.5) (layer B.Cu) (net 25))
 (segment (start 182.524 79.8322) (end 182.5244 79.8326) (width 0.25) (layer B.Cu) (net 8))
 (segment (start 182.5244 79.8326) (end 182.5244 81.28) (width 0.25) (layer B.Cu) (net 8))
 (segment (start 182.524 79.8322) (end 182.524 78.3844) (width 0.5) (layer B.Cu) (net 8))
 (segment (start 182.524 78.3844) (end 181.61 77.47) (width 0.5) (layer B.Cu) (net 8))
 (segment (start 182.524 81.28) (end 182.524 79.8322) (width 0.5) (layer B.Cu) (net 8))
 (segment (start 183.236 82.55) (end 183.2356 82.55) (width 0.25) (layer B.Cu) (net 24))
 (segment (start 183.236 82.55) (end 184.785 82.55) (width 0.5) (layer B.Cu) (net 24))
 (segment (start 182.524 82.55) (end 182.5244 82.55) (width 0.25) (layer B.Cu) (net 7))
 (segment (start 181.61 74.93) (end 180.34 76.2) (width 0.254) (layer B.Cu) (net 7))
 (segment (start 180.34 76.2) (end 180.34 81.915) (width 0.254) (layer B.Cu) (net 7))
 (segment (start 180.34 81.915) (end 180.975 82.55) (width 0.254) (layer B.Cu) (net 7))
 (segment (start 180.975 82.55) (end 182.524 82.55) (width 0.254) (layer B.Cu) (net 7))
 (segment (start 181.61 59.69) (end 181.61 49.53) (width 0.5) (layer F.Cu) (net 1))
 (segment (start 181.61 67.31) (end 183.134 67.31) (width 0.25) (layer F.Cu) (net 4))
 (segment (start 183.134 67.31) (end 186.69 63.754) (width 0.25) (layer F.Cu) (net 4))
 (segment (start 186.69 63.754) (end 186.69 49.53) (width 0.25) (layer F.Cu) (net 4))
 (segment (start 181.61 69.85) (end 186.182 69.85) (width 0.254) (layer F.Cu) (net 5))
 (segment (start 186.182 69.85) (end 188.468 72.136) (width 0.254) (layer F.Cu) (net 5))
 (segment (start 188.468 72.136) (end 188.468 87.376) (width 0.254) (layer F.Cu) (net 5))
 (segment (start 188.468 87.376) (end 184.912 90.932) (width 0.254) (layer F.Cu) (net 5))
 (segment (start 184.912 90.932) (end 184.912 99.314) (width 0.254) (layer F.Cu) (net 5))
 (segment (start 184.912 99.314) (end 186.69 101.092) (width 0.254) (layer F.Cu) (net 5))
 (segment (start 186.69 101.092) (end 196.088 101.092) (width 0.254) (layer F.Cu) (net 5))
 (segment (start 196.088 101.092) (end 198.04 103.044) (width 0.254) (layer F.Cu) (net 5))
 (segment (start 198.04 103.044) (end 198.04 108.465) (width 0.254) (layer F.Cu) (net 5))
 (segment (start 196.04 108.465) (end 196.04 102.822) (width 0.254) (layer F.Cu) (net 6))
 (segment (start 196.04 102.822) (end 194.818 101.6) (width 0.254) (layer F.Cu) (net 6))
 (segment (start 194.818 101.6) (end 186.436 101.6) (width 0.254) (layer F.Cu) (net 6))
 (segment (start 186.436 101.6) (end 184.404 99.568) (width 0.254) (layer F.Cu) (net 6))
 (segment (start 184.404 99.568) (end 184.404 90.678) (width 0.254) (layer F.Cu) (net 6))
 (segment (start 184.404 90.678) (end 187.96 87.122) (width 0.254) (layer F.Cu) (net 6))
 (segment (start 187.96 87.122) (end 187.96 74.676) (width 0.254) (layer F.Cu) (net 6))
 (segment (start 187.96 74.676) (end 185.674 72.39) (width 0.254) (layer F.Cu) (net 6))
 (segment (start 185.674 72.39) (end 181.61 72.39) (width 0.254) (layer F.Cu) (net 6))
 (segment (start 204.47 88.9) (end 204.47 87.884) (width 0.254) (layer B.Cu) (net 9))
 (segment (start 204.47 87.884) (end 205.486 86.868) (width 0.254) (layer B.Cu) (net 9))
 (segment (start 205.486 86.868) (end 205.486 78.486) (width 0.254) (layer B.Cu) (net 9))
 (segment (start 205.486 78.486) (end 204.47 77.47) (width 0.254) (layer B.Cu) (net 9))
 (segment (start 204.47 74.93) (end 205.74 73.66) (width 0.254) (layer F.Cu) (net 10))
 (segment (start 205.74 73.66) (end 205.74 50.8) (width 0.254) (layer F.Cu) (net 10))
 (segment (start 205.74 50.8) (end 204.47 49.53) (width 0.254) (layer F.Cu) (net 10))
 (segment (start 190.04 93.465) (end 190.04 75.644) (width 0.254) (layer F.Cu) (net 11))
 (segment (start 190.04 75.644) (end 193.294 72.39) (width 0.254) (layer F.Cu) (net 11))
 (segment (start 193.294 72.39) (end 204.47 72.39) (width 0.254) (layer B.Cu) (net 11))
 (via (at 193.294 72.39) (size 0.6) (layers F.Cu B.Cu) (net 11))
 (segment (start 195.326 70.104) (end 195.58 69.85) (width 0.254) (layer B.Cu) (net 12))
 (segment (start 195.58 69.85) (end 204.47 69.85) (width 0.254) (layer B.Cu) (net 12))
 (segment (start 194.04 93.465) (end 194.04 92.345) (width 0.254) (layer F.Cu) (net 12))
 (segment (start 194.04 92.345) (end 195.326 91.059) (width 0.254) (layer F.Cu) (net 12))
 (segment (start 195.326 91.059) (end 195.326 70.104) (width 0.254) (layer F.Cu) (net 12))
 (via (at 195.326 70.104) (size 0.6) (layers F.Cu B.Cu) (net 12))
 (segment (start 198.04 93.465) (end 198.04 69.295) (width 0.254) (layer F.Cu) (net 13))
 (segment (start 198.04 69.295) (end 200.025 67.31) (width 0.254) (layer F.Cu) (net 13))
 (segment (start 200.025 67.31) (end 204.47 67.31) (width 0.254) (layer F.Cu) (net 13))
 (segment (start 196.04 93.465) (end 196.04 67.485) (width 0.254) (layer F.Cu) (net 14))
 (segment (start 196.04 67.485) (end 198.755 64.77) (width 0.254) (layer F.Cu) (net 14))
 (segment (start 198.755 64.77) (end 204.47 64.77) (width 0.254) (layer F.Cu) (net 14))
 (segment (start 192.04 93.465) (end 192.04 92.186) (width 0.254) (layer F.Cu) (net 15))
 (segment (start 192.04 92.186) (end 194.564 89.662) (width 0.254) (layer F.Cu) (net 15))
 (segment (start 194.564 89.662) (end 194.564 66.548) (width 0.254) (layer F.Cu) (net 15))
 (segment (start 194.564 66.548) (end 198.882 62.23) (width 0.254) (layer F.Cu) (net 15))
 (segment (start 198.882 62.23) (end 204.47 62.23) (width 0.254) (layer F.Cu) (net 15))
 (segment (start 193.04 129.286) (end 193.04 130.048) (width 1.25) (layer F.Cu) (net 26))
 (segment (start 186.04 108.465) (end 186.04 111.11) (width 1.25) (layer F.Cu) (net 26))
 (segment (start 186.04 111.11) (end 188.722 113.792) (width 1.25) (layer F.Cu) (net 26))
 (segment (start 188.722 113.792) (end 192.024 113.792) (width 1.25) (layer F.Cu) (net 26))
 (segment (start 192.024 113.792) (end 193.04 114.808) (width 1.25) (layer F.Cu) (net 26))
 (segment (start 193.04 114.808) (end 193.04 129.286) (width 1.25) (layer F.Cu) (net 26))
 (segment (start 201.295 86.36) (end 196.088 86.36) (width 0.254) (layer B.Cu) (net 17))
 (segment (start 196.088 86.36) (end 196.088 88.9) (width 0.254) (layer B.Cu) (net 17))
 (segment (start 196.088 88.9) (end 198.12 90.932) (width 0.254) (layer B.Cu) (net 17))
 (segment (start 198.12 90.932) (end 203.708 90.932) (width 0.254) (layer B.Cu) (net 17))
 (segment (start 203.708 90.932) (end 205.42 92.644) (width 0.254) (layer B.Cu) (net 17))
 (segment (start 205.42 92.644) (end 205.42 93.98) (width 0.254) (layer B.Cu) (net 17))
 (segment (start 186.055 86.36) (end 182.372 86.36) (width 0.254) (layer F.Cu) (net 17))
 (segment (start 182.372 86.36) (end 180.594 84.582) (width 0.254) (layer F.Cu) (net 17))
 (segment (start 180.594 84.582) (end 180.66 84.648) (width 0.254) (layer B.Cu) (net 17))
 (segment (start 180.66 84.648) (end 180.66 85.725) (width 0.254) (layer B.Cu) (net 17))
 (segment (start 196.088 86.36) (end 186.055 86.36) (width 0.254) (layer B.Cu) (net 17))
 (via (at 180.594 84.582) (size 0.6) (layers F.Cu B.Cu) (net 17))
 (via (at 186.055 86.36) (size 0.6) (layers F.Cu B.Cu) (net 17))
 (segment (start 201.295 93.98) (end 203.52 93.98) (width 0.5) (layer B.Cu) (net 18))
 (segment (start 184.785 86.36) (end 183.515 86.36) (width 0.5) (layer B.Cu) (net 19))
 (segment (start 183.515 86.36) (end 182.88 85.725) (width 0.5) (layer B.Cu) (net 19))
 (segment (start 182.88 85.725) (end 182.56 85.725) (width 0.5) (layer B.Cu) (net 19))
 (segment (start 182.56 87.63) (end 184.785 87.63) (width 0.5) (layer B.Cu) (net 20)))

